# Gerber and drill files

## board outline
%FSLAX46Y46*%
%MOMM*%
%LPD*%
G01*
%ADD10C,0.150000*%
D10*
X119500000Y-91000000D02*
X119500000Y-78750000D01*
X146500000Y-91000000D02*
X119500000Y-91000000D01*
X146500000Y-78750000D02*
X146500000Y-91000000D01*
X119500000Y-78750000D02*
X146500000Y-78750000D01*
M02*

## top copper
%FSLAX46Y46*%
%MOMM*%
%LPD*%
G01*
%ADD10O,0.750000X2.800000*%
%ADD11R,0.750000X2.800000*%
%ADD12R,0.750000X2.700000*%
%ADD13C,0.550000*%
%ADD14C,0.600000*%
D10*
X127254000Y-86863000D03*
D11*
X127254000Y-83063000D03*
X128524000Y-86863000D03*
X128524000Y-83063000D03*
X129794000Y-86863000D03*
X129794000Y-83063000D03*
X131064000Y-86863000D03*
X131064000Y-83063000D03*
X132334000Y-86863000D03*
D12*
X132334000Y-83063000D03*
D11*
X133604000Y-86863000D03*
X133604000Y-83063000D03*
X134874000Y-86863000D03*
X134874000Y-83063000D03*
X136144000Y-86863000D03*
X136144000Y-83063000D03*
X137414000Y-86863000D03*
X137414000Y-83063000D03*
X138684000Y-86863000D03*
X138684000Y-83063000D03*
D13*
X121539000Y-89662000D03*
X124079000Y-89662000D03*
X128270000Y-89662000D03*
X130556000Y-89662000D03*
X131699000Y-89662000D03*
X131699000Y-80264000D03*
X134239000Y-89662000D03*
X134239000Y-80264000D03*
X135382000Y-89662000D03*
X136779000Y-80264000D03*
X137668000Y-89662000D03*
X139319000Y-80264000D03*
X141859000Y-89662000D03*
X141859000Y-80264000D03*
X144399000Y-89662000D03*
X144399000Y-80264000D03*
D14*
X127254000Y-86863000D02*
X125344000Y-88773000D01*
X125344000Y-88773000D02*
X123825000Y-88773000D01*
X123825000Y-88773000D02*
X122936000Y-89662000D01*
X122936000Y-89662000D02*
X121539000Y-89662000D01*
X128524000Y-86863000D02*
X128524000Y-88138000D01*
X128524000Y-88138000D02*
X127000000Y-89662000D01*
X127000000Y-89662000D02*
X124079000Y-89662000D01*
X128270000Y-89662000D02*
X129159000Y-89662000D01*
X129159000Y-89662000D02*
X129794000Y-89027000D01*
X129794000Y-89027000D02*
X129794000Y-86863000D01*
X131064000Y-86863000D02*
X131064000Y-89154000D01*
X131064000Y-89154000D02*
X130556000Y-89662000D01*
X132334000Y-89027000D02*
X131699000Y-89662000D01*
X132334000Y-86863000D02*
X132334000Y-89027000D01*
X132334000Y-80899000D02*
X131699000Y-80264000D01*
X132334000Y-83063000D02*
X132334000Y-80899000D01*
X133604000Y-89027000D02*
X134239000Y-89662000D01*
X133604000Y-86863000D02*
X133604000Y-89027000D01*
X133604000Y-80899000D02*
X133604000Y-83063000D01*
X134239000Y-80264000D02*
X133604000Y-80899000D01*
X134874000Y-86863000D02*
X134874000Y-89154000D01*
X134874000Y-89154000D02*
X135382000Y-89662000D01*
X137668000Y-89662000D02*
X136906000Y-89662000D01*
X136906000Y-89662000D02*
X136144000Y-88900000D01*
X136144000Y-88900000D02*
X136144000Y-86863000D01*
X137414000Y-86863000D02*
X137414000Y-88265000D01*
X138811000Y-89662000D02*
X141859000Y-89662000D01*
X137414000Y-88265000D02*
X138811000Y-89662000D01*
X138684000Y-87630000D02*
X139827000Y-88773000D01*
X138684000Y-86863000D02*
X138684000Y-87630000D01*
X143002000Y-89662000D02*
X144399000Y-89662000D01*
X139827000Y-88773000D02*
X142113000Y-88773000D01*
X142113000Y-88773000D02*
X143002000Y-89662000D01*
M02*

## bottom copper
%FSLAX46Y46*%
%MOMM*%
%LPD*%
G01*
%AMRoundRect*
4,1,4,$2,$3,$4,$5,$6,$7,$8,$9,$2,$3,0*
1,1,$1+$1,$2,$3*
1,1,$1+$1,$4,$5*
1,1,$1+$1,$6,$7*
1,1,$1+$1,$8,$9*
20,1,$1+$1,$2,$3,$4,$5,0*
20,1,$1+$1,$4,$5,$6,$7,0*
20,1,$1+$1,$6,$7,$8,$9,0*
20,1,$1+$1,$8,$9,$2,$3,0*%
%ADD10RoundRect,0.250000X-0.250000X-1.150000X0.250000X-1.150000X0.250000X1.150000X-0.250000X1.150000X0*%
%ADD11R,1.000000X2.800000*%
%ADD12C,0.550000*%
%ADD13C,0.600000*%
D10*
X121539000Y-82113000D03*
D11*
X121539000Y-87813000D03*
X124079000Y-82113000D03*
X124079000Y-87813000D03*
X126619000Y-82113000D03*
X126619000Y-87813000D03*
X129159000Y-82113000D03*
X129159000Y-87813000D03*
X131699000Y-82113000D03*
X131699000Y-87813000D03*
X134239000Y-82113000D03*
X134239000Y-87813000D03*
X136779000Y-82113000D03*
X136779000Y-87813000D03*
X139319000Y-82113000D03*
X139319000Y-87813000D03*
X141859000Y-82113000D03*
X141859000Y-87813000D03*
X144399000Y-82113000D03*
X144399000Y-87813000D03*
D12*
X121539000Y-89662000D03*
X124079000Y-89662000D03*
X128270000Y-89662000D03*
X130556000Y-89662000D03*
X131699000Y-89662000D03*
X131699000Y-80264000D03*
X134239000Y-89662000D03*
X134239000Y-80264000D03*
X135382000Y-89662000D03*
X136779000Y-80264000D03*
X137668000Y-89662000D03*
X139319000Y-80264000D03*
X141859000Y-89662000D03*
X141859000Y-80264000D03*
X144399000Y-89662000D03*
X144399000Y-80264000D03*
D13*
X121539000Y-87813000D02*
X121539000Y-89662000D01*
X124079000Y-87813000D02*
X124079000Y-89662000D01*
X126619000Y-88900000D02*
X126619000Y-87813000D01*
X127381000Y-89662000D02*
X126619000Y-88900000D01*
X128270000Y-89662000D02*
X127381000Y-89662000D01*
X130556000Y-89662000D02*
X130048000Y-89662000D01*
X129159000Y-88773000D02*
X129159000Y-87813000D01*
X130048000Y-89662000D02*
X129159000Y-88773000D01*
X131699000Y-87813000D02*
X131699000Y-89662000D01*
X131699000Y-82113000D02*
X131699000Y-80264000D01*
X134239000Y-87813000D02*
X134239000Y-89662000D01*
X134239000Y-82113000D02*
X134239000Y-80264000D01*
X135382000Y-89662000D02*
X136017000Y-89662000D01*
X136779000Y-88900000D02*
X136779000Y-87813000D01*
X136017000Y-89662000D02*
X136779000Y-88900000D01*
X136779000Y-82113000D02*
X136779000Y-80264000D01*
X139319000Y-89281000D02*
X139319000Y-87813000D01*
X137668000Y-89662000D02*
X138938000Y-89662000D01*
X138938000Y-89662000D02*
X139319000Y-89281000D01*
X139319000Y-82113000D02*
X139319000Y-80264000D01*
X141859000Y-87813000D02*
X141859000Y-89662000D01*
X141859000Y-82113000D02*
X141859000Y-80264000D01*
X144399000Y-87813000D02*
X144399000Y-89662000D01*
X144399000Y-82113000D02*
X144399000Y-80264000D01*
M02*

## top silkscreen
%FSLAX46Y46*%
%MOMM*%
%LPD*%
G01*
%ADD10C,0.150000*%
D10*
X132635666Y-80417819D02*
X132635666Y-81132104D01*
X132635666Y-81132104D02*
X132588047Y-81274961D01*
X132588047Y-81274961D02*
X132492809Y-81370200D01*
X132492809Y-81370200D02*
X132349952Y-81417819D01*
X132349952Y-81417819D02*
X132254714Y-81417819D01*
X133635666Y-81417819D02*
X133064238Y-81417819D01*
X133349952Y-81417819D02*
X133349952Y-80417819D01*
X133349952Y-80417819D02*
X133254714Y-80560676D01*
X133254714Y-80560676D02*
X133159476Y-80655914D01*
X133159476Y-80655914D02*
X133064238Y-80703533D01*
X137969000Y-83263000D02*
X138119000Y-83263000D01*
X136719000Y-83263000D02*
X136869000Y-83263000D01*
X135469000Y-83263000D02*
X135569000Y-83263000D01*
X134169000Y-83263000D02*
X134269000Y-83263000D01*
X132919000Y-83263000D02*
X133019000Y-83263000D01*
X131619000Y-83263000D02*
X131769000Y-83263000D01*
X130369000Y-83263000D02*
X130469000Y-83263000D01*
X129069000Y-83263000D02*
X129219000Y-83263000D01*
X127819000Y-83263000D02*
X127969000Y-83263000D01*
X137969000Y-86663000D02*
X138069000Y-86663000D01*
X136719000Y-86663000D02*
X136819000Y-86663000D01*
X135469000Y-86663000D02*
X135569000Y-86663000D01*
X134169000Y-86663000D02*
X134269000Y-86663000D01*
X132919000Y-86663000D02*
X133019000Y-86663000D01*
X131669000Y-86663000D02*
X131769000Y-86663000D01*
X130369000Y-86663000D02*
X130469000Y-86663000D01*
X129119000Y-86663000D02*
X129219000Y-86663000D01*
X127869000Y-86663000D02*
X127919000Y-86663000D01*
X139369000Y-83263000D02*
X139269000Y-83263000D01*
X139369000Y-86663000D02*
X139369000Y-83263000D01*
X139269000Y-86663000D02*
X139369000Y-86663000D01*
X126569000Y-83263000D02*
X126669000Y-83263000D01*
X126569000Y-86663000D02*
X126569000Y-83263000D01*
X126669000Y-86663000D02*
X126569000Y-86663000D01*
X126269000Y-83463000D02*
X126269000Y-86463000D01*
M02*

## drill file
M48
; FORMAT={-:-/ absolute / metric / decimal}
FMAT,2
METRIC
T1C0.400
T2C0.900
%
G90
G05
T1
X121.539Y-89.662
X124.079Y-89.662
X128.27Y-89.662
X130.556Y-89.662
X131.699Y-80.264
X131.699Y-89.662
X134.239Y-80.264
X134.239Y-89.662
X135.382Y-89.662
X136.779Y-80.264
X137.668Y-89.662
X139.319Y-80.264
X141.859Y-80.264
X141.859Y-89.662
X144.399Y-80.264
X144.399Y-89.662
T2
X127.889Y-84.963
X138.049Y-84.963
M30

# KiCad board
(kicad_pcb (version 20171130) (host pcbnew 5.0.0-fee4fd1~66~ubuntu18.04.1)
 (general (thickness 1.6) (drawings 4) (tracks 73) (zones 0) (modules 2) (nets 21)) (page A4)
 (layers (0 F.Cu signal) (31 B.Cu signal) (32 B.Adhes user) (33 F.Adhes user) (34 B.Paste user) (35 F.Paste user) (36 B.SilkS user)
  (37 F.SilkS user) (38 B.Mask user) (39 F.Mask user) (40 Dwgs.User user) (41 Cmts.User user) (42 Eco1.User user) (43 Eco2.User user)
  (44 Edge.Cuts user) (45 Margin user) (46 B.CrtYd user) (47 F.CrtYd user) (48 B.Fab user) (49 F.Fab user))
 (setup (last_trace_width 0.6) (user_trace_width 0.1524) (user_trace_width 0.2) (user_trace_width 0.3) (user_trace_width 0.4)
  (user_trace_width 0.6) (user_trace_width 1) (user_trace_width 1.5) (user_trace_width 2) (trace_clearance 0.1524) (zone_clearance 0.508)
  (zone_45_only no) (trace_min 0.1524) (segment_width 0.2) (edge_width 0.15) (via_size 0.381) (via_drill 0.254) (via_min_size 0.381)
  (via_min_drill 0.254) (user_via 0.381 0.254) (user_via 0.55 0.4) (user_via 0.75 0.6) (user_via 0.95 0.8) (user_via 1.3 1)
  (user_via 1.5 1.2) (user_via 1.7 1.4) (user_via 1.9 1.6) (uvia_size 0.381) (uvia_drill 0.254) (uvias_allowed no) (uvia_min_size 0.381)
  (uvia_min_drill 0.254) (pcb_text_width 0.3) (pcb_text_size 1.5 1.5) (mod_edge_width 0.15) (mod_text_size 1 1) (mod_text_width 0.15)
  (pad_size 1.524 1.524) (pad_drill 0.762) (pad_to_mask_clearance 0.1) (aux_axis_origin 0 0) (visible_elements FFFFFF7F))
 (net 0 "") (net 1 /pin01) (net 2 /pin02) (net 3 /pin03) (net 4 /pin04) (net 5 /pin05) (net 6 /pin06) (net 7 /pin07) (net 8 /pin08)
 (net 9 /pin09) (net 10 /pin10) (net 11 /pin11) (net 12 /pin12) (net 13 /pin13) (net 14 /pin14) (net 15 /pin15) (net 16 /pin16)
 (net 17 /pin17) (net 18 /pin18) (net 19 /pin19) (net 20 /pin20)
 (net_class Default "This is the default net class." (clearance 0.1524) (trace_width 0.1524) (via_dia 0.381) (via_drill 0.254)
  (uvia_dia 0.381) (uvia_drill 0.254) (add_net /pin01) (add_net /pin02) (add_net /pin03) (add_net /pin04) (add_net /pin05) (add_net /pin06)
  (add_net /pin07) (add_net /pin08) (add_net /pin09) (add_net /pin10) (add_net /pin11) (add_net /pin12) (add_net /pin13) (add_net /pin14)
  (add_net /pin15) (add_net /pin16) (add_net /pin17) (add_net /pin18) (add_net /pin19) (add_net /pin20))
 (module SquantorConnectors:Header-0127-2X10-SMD (layer F.Cu) (at 132.969 84.963)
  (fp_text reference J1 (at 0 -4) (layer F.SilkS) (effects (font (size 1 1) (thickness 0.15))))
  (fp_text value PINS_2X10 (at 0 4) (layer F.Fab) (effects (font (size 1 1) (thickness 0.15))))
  (fp_line (start 5 -1.7) (end 5.15 -1.7) (layer F.SilkS) (width 0.15))
  (fp_line (start 3.75 -1.7) (end 3.9 -1.7) (layer F.SilkS) (width 0.15))
  (fp_line (start 2.5 -1.7) (end 2.6 -1.7) (layer F.SilkS) (width 0.15))
  (fp_line (start 1.2 -1.7) (end 1.3 -1.7) (layer F.SilkS) (width 0.15))
  (fp_line (start -0.05 -1.7) (end 0.05 -1.7) (layer F.SilkS) (width 0.15))
  (fp_line (start -1.35 -1.7) (end -1.2 -1.7) (layer F.SilkS) (width 0.15))
  (fp_line (start -2.6 -1.7) (end -2.5 -1.7) (layer F.SilkS) (width 0.15))
  (fp_line (start -3.9 -1.7) (end -3.75 -1.7) (layer F.SilkS) (width 0.15))
  (fp_line (start -5.15 -1.7) (end -5 -1.7) (layer F.SilkS) (width 0.15))
  (fp_line (start 5 1.7) (end 5.1 1.7) (layer F.SilkS) (width 0.15))
  (fp_line (start 3.75 1.7) (end 3.85 1.7) (layer F.SilkS) (width 0.15))
  (fp_line (start 2.5 1.7) (end 2.6 1.7) (layer F.SilkS) (width 0.15))
  (fp_line (start 1.2 1.7) (end 1.3 1.7) (layer F.SilkS) (width 0.15))
  (fp_line (start -0.05 1.7) (end 0.05 1.7) (layer F.SilkS) (width 0.15))
  (fp_line (start -1.3 1.7) (end -1.2 1.7) (layer F.SilkS) (width 0.15))
  (fp_line (start -2.6 1.7) (end -2.5 1.7) (layer F.SilkS) (width 0.15))
  (fp_line (start -3.85 1.7) (end -3.75 1.7) (layer F.SilkS) (width 0.15))
  (fp_line (start -5.1 1.7) (end -5.05 1.7) (layer F.SilkS) (width 0.15))
  (fp_line (start 6.4 -1.7) (end 6.3 -1.7) (layer F.SilkS) (width 0.15))
  (fp_line (start 6.4 1.7) (end 6.4 -1.7) (layer F.SilkS) (width 0.15))
  (fp_line (start 6.3 1.7) (end 6.4 1.7) (layer F.SilkS) (width 0.15))
  (fp_line (start -6.4 -1.7) (end -6.3 -1.7) (layer F.SilkS) (width 0.15))
  (fp_line (start -6.4 1.7) (end -6.4 -1.7) (layer F.SilkS) (width 0.15))
  (fp_line (start -6.3 1.7) (end -6.4 1.7) (layer F.SilkS) (width 0.15))
  (fp_line (start -6.7 -1.5) (end -6.7 1.5) (layer F.SilkS) (width 0.15))
  (pad 1 smd oval (at -5.715 1.9) (size 0.75 2.8) (layers F.Cu F.Paste F.Mask) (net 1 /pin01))
  (pad 2 smd rect (at -5.715 -1.9) (size 0.75 2.8) (layers F.Cu F.Paste F.Mask) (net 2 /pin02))
  (pad 3 smd rect (at -4.445 1.9) (size 0.75 2.8) (layers F.Cu F.Paste F.Mask) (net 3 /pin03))
  (pad 4 smd rect (at -4.445 -1.9) (size 0.75 2.8) (layers F.Cu F.Paste F.Mask) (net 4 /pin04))
  (pad 5 smd rect (at -3.175 1.9) (size 0.75 2.8) (layers F.Cu F.Paste F.Mask) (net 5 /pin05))
  (pad 6 smd rect (at -3.175 -1.9) (size 0.75 2.8) (layers F.Cu F.Paste F.Mask) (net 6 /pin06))
  (pad 7 smd rect (at -1.905 1.9) (size 0.75 2.8) (layers F.Cu F.Paste F.Mask) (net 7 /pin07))
  (pad 8 smd rect (at -1.905 -1.9) (size 0.75 2.8) (layers F.Cu F.Paste F.Mask) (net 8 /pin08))
  (pad 9 smd rect (at -0.635 1.9) (size 0.75 2.8) (layers F.Cu F.Paste F.Mask) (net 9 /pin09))
  (pad 10 smd rect (at -0.635 -1.9) (size 0.75 2.7) (layers F.Cu F.Paste F.Mask) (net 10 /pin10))
  (pad 11 smd rect (at 0.635 1.9) (size 0.75 2.8) (layers F.Cu F.Paste F.Mask) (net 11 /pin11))
  (pad 12 smd rect (at 0.635 -1.9) (size 0.75 2.8) (layers F.Cu F.Paste F.Mask) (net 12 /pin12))
  (pad 13 smd rect (at 1.905 1.9) (size 0.75 2.8) (layers F.Cu F.Paste F.Mask) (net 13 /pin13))
  (pad 14 smd rect (at 1.905 -1.9) (size 0.75 2.8) (layers F.Cu F.Paste F.Mask) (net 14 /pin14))
  (pad 15 smd rect (at 3.175 1.9) (size 0.75 2.8) (layers F.Cu F.Paste F.Mask) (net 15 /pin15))
  (pad 16 smd rect (at 3.175 -1.9) (size 0.75 2.8) (layers F.Cu F.Paste F.Mask) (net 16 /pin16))
  (pad 17 smd rect (at 4.445 1.9) (size 0.75 2.8) (layers F.Cu F.Paste F.Mask) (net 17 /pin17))
  (pad 18 smd rect (at 4.445 -1.9) (size 0.75 2.8) (layers F.Cu F.Paste F.Mask) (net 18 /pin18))
  (pad 19 smd rect (at 5.715 1.9) (size 0.75 2.8) (layers F.Cu F.Paste F.Mask) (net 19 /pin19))
  (pad 20 smd rect (at 5.715 -1.9) (size 0.75 2.8) (layers F.Cu F.Paste F.Mask) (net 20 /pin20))
  (pad "" np_thru_hole circle (at -5.08 0) (size 0.9 0.9) (drill 0.9) (layers *.Cu *.Mask))
  (pad "" np_thru_hole circle (at 5.08 0) (size 0.9 0.9) (drill 0.9) (layers *.Cu *.Mask)))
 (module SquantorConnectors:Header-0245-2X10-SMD (layer B.Cu) (at 132.969 84.963)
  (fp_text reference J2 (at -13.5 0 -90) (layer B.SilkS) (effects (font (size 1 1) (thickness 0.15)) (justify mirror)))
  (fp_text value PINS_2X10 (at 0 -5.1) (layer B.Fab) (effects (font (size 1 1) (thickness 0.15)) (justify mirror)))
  (pad 1 smd roundrect (at -11.43 -2.85) (size 1 2.8) (layers B.Cu B.Paste B.Mask) (roundrect_rratio 0.25) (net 2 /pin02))
  (pad 2 smd rect (at -11.43 2.85) (size 1 2.8) (layers B.Cu B.Paste B.Mask) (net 1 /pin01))
  (pad 3 smd rect (at -8.89 -2.85) (size 1 2.8) (layers B.Cu B.Paste B.Mask) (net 4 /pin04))
  (pad 4 smd rect (at -8.89 2.85) (size 1 2.8) (layers B.Cu B.Paste B.Mask) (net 3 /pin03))
  (pad 5 smd rect (at -6.35 -2.85) (size 1 2.8) (layers B.Cu B.Paste B.Mask) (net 6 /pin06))
  (pad 6 smd rect (at -6.35 2.85) (size 1 2.8) (layers B.Cu B.Paste B.Mask) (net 5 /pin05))
  (pad 7 smd rect (at -3.81 -2.85) (size 1 2.8) (layers B.Cu B.Paste B.Mask) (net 8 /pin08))
  (pad 8 smd rect (at -3.81 2.85) (size 1 2.8) (layers B.Cu B.Paste B.Mask) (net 7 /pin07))
  (pad 9 smd rect (at -1.27 -2.85) (size 1 2.8) (layers B.Cu B.Paste B.Mask) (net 10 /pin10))
  (pad 10 smd rect (at -1.27 2.85) (size 1 2.8) (layers B.Cu B.Paste B.Mask) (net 9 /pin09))
  (pad 11 smd rect (at 1.27 -2.85) (size 1 2.8) (layers B.Cu B.Paste B.Mask) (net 12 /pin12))
  (pad 12 smd rect (at 1.27 2.85) (size 1 2.8) (layers B.Cu B.Paste B.Mask) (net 11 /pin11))
  (pad 13 smd rect (at 3.81 -2.85) (size 1 2.8) (layers B.Cu B.Paste B.Mask) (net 14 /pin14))
  (pad 14 smd rect (at 3.81 2.85) (size 1 2.8) (layers B.Cu B.Paste B.Mask) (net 13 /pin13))
  (pad 15 smd rect (at 6.35 -2.85) (size 1 2.8) (layers B.Cu B.Paste B.Mask) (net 16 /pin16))
  (pad 16 smd rect (at 6.35 2.85) (size 1 2.8) (layers B.Cu B.Paste B.Mask) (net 15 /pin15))
  (pad 17 smd rect (at 8.89 -2.85) (size 1 2.8) (layers B.Cu B.Paste B.Mask) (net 18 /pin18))
  (pad 18 smd rect (at 8.89 2.85) (size 1 2.8) (layers B.Cu B.Paste B.Mask) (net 17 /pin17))
  (pad 19 smd rect (at 11.43 -2.85) (size 1 2.8) (layers B.Cu B.Paste B.Mask) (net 20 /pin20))
  (pad 20 smd rect (at 11.43 2.85) (size 1 2.8) (layers B.Cu B.Paste B.Mask) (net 19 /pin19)))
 (gr_line (start 119.5 91) (end 119.5 78.75) (layer Edge.Cuts) (width 0.15))
 (gr_line (start 146.5 91) (end 119.5 91) (layer Edge.Cuts) (width 0.15))
 (gr_line (start 146.5 78.75) (end 146.5 91) (layer Edge.Cuts) (width 0.15))
 (gr_line (start 119.5 78.75) (end 146.5 78.75) (layer Edge.Cuts) (width 0.15))
 (segment (start 127.254 86.863) (end 125.344 88.773) (width 0.6) (layer F.Cu) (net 1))
 (segment (start 125.344 88.773) (end 123.825 88.773) (width 0.6) (layer F.Cu) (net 1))
 (segment (start 123.825 88.773) (end 122.936 89.662) (width 0.6) (layer F.Cu) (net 1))
 (via (at 121.539 89.662) (size 0.55) (drill 0.4) (layers F.Cu B.Cu) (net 1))
 (segment (start 122.936 89.662) (end 121.539 89.662) (width 0.6) (layer F.Cu) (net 1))
 (segment (start 121.539 87.813) (end 121.539 89.662) (width 0.6) (layer B.Cu) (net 1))
 (segment (start 128.524 86.863) (end 128.524 88.138) (width 0.6) (layer F.Cu) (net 3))
 (segment (start 128.524 88.138) (end 127 89.662) (width 0.6) (layer F.Cu) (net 3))
 (via (at 124.079 89.662) (size 0.55) (drill 0.4) (layers F.Cu B.Cu) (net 3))
 (segment (start 127 89.662) (end 124.079 89.662) (width 0.6) (layer F.Cu) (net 3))
 (segment (start 124.079 87.813) (end 124.079 89.662) (width 0.6) (layer B.Cu) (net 3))
 (segment (start 126.619 88.9) (end 126.619 87.813) (width 0.6) (layer B.Cu) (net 5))
 (segment (start 128.27 89.662) (end 129.159 89.662) (width 0.6) (layer F.Cu) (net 5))
 (segment (start 129.159 89.662) (end 129.794 89.027) (width 0.6) (layer F.Cu) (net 5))
 (via (at 128.27 89.662) (size 0.55) (drill 0.4) (layers F.Cu B.Cu) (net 5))
 (segment (start 129.794 89.027) (end 129.794 86.863) (width 0.6) (layer F.Cu) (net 5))
 (segment (start 127.381 89.662) (end 126.619 88.9) (width 0.6) (layer B.Cu) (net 5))
 (segment (start 128.27 89.662) (end 127.381 89.662) (width 0.6) (layer B.Cu) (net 5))
 (segment (start 131.064 86.863) (end 131.064 89.154) (width 0.6) (layer F.Cu) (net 7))
 (via (at 130.556 89.662) (size 0.55) (drill 0.4) (layers F.Cu B.Cu) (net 7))
 (segment (start 131.064 89.154) (end 130.556 89.662) (width 0.6) (layer F.Cu) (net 7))
 (segment (start 130.556 89.662) (end 130.048 89.662) (width 0.6) (layer B.Cu) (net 7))
 (segment (start 129.159 88.773) (end 129.159 87.813) (width 0.6) (layer B.Cu) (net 7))
 (segment (start 130.048 89.662) (end 129.159 88.773) (width 0.6) (layer B.Cu) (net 7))
 (via (at 131.699 89.662) (size 0.55) (drill 0.4) (layers F.Cu B.Cu) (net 9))
 (segment (start 131.699 87.813) (end 131.699 89.662) (width 0.6) (layer B.Cu) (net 9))
 (segment (start 132.334 89.027) (end 131.699 89.662) (width 0.6) (layer F.Cu) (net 9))
 (segment (start 132.334 86.863) (end 132.334 89.027) (width 0.6) (layer F.Cu) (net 9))
 (via (at 131.699 80.264) (size 0.55) (drill 0.4) (layers F.Cu B.Cu) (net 10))
 (segment (start 131.699 82.113) (end 131.699 80.264) (width 0.6) (layer B.Cu) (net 10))
 (segment (start 132.334 80.899) (end 131.699 80.264) (width 0.6) (layer F.Cu) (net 10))
 (segment (start 132.334 83.063) (end 132.334 80.899) (width 0.6) (layer F.Cu) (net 10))
 (via (at 134.239 89.662) (size 0.55) (drill 0.4) (layers F.Cu B.Cu) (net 11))
 (segment (start 134.239 87.813) (end 134.239 89.662) (width 0.6) (layer B.Cu) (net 11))
 (segment (start 133.604 89.027) (end 134.239 89.662) (width 0.6) (layer F.Cu) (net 11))
 (segment (start 133.604 86.863) (end 133.604 89.027) (width 0.6) (layer F.Cu) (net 11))
 (via (at 134.239 80.264) (size 0.55) (drill 0.4) (layers F.Cu B.Cu) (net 12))
 (segment (start 134.239 82.113) (end 134.239 80.264) (width 0.6) (layer B.Cu) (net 12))
 (segment (start 133.604 80.899) (end 133.604 83.063) (width 0.6) (layer F.Cu) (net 12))
 (segment (start 134.239 80.264) (end 133.604 80.899) (width 0.6) (layer F.Cu) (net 12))
 (segment (start 134.874 86.863) (end 134.874 89.154) (width 0.6) (layer F.Cu) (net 13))
 (via (at 135.382 89.662) (size 0.55) (drill 0.4) (layers F.Cu B.Cu) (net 13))
 (segment (start 134.874 89.154) (end 135.382 89.662) (width 0.6) (layer F.Cu) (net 13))
 (segment (start 135.382 89.662) (end 136.017 89.662) (width 0.6) (layer B.Cu) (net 13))
 (segment (start 136.779 88.9) (end 136.779 87.813) (width 0.6) (layer B.Cu) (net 13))
 (segment (start 136.017 89.662) (end 136.779 88.9) (width 0.6) (layer B.Cu) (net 13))
 (via (at 136.779 80.264) (size 0.55) (drill 0.4) (layers F.Cu B.Cu) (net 14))
 (segment (start 136.779 82.113) (end 136.779 80.264) (width 0.6) (layer B.Cu) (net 14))
 (segment (start 139.319 89.281) (end 139.319 87.813) (width 0.6) (layer B.Cu) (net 15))
 (segment (start 137.668 89.662) (end 136.906 89.662) (width 0.6) (layer F.Cu) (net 15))
 (segment (start 136.906 89.662) (end 136.144 88.9) (width 0.6) (layer F.Cu) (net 15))
 (via (at 137.668 89.662) (size 0.55) (drill 0.4) (layers F.Cu B.Cu) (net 15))
 (segment (start 136.144 88.9) (end 136.144 86.863) (width 0.6) (layer F.Cu) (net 15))
 (segment (start 137.668 89.662) (end 138.938 89.662) (width 0.6) (layer B.Cu) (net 15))
 (segment (start 138.938 89.662) (end 139.319 89.281) (width 0.6) (layer B.Cu) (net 15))
 (via (at 139.319 80.264) (size 0.55) (drill 0.4) (layers F.Cu B.Cu) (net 16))
 (segment (start 139.319 82.113) (end 139.319 80.264) (width 0.6) (layer B.Cu) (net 16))
 (via (at 141.859 89.662) (size 0.55) (drill 0.4) (layers F.Cu B.Cu) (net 17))
 (segment (start 141.859 87.813) (end 141.859 89.662) (width 0.6) (layer B.Cu) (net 17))
 (segment (start 137.414 86.863) (end 137.414 88.265) (width 0.6) (layer F.Cu) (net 17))
 (segment (start 138.811 89.662) (end 141.859 89.662) (width 0.6) (layer F.Cu) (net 17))
 (segment (start 137.414 88.265) (end 138.811 89.662) (width 0.6) (layer F.Cu) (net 17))
 (via (at 141.859 80.264) (size 0.55) (drill 0.4) (layers F.Cu B.Cu) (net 18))
 (segment (start 141.859 82.113) (end 141.859 80.264) (width 0.6) (layer B.Cu) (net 18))
 (via (at 144.399 89.662) (size 0.55) (drill 0.4) (layers F.Cu B.Cu) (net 19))
 (segment (start 144.399 87.813) (end 144.399 89.662) (width 0.6) (layer B.Cu) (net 19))
 (segment (start 138.684 87.63) (end 139.827 88.773) (width 0.6) (layer F.Cu) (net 19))
 (segment (start 138.684 86.863) (end 138.684 87.63) (width 0.6) (layer F.Cu) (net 19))
 (segment (start 143.002 89.662) (end 144.399 89.662) (width 0.6) (layer F.Cu) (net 19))
 (segment (start 139.827 88.773) (end 142.113 88.773) (width 0.6) (layer F.Cu) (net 19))
 (segment (start 142.113 88.773) (end 143.002 89.662) (width 0.6) (layer F.Cu) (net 19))
 (via (at 144.399 80.264) (size 0.55) (drill 0.4) (layers F.Cu B.Cu) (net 20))
 (segment (start 144.399 82.113) (end 144.399 80.264) (width 0.6) (layer B.Cu) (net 20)))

